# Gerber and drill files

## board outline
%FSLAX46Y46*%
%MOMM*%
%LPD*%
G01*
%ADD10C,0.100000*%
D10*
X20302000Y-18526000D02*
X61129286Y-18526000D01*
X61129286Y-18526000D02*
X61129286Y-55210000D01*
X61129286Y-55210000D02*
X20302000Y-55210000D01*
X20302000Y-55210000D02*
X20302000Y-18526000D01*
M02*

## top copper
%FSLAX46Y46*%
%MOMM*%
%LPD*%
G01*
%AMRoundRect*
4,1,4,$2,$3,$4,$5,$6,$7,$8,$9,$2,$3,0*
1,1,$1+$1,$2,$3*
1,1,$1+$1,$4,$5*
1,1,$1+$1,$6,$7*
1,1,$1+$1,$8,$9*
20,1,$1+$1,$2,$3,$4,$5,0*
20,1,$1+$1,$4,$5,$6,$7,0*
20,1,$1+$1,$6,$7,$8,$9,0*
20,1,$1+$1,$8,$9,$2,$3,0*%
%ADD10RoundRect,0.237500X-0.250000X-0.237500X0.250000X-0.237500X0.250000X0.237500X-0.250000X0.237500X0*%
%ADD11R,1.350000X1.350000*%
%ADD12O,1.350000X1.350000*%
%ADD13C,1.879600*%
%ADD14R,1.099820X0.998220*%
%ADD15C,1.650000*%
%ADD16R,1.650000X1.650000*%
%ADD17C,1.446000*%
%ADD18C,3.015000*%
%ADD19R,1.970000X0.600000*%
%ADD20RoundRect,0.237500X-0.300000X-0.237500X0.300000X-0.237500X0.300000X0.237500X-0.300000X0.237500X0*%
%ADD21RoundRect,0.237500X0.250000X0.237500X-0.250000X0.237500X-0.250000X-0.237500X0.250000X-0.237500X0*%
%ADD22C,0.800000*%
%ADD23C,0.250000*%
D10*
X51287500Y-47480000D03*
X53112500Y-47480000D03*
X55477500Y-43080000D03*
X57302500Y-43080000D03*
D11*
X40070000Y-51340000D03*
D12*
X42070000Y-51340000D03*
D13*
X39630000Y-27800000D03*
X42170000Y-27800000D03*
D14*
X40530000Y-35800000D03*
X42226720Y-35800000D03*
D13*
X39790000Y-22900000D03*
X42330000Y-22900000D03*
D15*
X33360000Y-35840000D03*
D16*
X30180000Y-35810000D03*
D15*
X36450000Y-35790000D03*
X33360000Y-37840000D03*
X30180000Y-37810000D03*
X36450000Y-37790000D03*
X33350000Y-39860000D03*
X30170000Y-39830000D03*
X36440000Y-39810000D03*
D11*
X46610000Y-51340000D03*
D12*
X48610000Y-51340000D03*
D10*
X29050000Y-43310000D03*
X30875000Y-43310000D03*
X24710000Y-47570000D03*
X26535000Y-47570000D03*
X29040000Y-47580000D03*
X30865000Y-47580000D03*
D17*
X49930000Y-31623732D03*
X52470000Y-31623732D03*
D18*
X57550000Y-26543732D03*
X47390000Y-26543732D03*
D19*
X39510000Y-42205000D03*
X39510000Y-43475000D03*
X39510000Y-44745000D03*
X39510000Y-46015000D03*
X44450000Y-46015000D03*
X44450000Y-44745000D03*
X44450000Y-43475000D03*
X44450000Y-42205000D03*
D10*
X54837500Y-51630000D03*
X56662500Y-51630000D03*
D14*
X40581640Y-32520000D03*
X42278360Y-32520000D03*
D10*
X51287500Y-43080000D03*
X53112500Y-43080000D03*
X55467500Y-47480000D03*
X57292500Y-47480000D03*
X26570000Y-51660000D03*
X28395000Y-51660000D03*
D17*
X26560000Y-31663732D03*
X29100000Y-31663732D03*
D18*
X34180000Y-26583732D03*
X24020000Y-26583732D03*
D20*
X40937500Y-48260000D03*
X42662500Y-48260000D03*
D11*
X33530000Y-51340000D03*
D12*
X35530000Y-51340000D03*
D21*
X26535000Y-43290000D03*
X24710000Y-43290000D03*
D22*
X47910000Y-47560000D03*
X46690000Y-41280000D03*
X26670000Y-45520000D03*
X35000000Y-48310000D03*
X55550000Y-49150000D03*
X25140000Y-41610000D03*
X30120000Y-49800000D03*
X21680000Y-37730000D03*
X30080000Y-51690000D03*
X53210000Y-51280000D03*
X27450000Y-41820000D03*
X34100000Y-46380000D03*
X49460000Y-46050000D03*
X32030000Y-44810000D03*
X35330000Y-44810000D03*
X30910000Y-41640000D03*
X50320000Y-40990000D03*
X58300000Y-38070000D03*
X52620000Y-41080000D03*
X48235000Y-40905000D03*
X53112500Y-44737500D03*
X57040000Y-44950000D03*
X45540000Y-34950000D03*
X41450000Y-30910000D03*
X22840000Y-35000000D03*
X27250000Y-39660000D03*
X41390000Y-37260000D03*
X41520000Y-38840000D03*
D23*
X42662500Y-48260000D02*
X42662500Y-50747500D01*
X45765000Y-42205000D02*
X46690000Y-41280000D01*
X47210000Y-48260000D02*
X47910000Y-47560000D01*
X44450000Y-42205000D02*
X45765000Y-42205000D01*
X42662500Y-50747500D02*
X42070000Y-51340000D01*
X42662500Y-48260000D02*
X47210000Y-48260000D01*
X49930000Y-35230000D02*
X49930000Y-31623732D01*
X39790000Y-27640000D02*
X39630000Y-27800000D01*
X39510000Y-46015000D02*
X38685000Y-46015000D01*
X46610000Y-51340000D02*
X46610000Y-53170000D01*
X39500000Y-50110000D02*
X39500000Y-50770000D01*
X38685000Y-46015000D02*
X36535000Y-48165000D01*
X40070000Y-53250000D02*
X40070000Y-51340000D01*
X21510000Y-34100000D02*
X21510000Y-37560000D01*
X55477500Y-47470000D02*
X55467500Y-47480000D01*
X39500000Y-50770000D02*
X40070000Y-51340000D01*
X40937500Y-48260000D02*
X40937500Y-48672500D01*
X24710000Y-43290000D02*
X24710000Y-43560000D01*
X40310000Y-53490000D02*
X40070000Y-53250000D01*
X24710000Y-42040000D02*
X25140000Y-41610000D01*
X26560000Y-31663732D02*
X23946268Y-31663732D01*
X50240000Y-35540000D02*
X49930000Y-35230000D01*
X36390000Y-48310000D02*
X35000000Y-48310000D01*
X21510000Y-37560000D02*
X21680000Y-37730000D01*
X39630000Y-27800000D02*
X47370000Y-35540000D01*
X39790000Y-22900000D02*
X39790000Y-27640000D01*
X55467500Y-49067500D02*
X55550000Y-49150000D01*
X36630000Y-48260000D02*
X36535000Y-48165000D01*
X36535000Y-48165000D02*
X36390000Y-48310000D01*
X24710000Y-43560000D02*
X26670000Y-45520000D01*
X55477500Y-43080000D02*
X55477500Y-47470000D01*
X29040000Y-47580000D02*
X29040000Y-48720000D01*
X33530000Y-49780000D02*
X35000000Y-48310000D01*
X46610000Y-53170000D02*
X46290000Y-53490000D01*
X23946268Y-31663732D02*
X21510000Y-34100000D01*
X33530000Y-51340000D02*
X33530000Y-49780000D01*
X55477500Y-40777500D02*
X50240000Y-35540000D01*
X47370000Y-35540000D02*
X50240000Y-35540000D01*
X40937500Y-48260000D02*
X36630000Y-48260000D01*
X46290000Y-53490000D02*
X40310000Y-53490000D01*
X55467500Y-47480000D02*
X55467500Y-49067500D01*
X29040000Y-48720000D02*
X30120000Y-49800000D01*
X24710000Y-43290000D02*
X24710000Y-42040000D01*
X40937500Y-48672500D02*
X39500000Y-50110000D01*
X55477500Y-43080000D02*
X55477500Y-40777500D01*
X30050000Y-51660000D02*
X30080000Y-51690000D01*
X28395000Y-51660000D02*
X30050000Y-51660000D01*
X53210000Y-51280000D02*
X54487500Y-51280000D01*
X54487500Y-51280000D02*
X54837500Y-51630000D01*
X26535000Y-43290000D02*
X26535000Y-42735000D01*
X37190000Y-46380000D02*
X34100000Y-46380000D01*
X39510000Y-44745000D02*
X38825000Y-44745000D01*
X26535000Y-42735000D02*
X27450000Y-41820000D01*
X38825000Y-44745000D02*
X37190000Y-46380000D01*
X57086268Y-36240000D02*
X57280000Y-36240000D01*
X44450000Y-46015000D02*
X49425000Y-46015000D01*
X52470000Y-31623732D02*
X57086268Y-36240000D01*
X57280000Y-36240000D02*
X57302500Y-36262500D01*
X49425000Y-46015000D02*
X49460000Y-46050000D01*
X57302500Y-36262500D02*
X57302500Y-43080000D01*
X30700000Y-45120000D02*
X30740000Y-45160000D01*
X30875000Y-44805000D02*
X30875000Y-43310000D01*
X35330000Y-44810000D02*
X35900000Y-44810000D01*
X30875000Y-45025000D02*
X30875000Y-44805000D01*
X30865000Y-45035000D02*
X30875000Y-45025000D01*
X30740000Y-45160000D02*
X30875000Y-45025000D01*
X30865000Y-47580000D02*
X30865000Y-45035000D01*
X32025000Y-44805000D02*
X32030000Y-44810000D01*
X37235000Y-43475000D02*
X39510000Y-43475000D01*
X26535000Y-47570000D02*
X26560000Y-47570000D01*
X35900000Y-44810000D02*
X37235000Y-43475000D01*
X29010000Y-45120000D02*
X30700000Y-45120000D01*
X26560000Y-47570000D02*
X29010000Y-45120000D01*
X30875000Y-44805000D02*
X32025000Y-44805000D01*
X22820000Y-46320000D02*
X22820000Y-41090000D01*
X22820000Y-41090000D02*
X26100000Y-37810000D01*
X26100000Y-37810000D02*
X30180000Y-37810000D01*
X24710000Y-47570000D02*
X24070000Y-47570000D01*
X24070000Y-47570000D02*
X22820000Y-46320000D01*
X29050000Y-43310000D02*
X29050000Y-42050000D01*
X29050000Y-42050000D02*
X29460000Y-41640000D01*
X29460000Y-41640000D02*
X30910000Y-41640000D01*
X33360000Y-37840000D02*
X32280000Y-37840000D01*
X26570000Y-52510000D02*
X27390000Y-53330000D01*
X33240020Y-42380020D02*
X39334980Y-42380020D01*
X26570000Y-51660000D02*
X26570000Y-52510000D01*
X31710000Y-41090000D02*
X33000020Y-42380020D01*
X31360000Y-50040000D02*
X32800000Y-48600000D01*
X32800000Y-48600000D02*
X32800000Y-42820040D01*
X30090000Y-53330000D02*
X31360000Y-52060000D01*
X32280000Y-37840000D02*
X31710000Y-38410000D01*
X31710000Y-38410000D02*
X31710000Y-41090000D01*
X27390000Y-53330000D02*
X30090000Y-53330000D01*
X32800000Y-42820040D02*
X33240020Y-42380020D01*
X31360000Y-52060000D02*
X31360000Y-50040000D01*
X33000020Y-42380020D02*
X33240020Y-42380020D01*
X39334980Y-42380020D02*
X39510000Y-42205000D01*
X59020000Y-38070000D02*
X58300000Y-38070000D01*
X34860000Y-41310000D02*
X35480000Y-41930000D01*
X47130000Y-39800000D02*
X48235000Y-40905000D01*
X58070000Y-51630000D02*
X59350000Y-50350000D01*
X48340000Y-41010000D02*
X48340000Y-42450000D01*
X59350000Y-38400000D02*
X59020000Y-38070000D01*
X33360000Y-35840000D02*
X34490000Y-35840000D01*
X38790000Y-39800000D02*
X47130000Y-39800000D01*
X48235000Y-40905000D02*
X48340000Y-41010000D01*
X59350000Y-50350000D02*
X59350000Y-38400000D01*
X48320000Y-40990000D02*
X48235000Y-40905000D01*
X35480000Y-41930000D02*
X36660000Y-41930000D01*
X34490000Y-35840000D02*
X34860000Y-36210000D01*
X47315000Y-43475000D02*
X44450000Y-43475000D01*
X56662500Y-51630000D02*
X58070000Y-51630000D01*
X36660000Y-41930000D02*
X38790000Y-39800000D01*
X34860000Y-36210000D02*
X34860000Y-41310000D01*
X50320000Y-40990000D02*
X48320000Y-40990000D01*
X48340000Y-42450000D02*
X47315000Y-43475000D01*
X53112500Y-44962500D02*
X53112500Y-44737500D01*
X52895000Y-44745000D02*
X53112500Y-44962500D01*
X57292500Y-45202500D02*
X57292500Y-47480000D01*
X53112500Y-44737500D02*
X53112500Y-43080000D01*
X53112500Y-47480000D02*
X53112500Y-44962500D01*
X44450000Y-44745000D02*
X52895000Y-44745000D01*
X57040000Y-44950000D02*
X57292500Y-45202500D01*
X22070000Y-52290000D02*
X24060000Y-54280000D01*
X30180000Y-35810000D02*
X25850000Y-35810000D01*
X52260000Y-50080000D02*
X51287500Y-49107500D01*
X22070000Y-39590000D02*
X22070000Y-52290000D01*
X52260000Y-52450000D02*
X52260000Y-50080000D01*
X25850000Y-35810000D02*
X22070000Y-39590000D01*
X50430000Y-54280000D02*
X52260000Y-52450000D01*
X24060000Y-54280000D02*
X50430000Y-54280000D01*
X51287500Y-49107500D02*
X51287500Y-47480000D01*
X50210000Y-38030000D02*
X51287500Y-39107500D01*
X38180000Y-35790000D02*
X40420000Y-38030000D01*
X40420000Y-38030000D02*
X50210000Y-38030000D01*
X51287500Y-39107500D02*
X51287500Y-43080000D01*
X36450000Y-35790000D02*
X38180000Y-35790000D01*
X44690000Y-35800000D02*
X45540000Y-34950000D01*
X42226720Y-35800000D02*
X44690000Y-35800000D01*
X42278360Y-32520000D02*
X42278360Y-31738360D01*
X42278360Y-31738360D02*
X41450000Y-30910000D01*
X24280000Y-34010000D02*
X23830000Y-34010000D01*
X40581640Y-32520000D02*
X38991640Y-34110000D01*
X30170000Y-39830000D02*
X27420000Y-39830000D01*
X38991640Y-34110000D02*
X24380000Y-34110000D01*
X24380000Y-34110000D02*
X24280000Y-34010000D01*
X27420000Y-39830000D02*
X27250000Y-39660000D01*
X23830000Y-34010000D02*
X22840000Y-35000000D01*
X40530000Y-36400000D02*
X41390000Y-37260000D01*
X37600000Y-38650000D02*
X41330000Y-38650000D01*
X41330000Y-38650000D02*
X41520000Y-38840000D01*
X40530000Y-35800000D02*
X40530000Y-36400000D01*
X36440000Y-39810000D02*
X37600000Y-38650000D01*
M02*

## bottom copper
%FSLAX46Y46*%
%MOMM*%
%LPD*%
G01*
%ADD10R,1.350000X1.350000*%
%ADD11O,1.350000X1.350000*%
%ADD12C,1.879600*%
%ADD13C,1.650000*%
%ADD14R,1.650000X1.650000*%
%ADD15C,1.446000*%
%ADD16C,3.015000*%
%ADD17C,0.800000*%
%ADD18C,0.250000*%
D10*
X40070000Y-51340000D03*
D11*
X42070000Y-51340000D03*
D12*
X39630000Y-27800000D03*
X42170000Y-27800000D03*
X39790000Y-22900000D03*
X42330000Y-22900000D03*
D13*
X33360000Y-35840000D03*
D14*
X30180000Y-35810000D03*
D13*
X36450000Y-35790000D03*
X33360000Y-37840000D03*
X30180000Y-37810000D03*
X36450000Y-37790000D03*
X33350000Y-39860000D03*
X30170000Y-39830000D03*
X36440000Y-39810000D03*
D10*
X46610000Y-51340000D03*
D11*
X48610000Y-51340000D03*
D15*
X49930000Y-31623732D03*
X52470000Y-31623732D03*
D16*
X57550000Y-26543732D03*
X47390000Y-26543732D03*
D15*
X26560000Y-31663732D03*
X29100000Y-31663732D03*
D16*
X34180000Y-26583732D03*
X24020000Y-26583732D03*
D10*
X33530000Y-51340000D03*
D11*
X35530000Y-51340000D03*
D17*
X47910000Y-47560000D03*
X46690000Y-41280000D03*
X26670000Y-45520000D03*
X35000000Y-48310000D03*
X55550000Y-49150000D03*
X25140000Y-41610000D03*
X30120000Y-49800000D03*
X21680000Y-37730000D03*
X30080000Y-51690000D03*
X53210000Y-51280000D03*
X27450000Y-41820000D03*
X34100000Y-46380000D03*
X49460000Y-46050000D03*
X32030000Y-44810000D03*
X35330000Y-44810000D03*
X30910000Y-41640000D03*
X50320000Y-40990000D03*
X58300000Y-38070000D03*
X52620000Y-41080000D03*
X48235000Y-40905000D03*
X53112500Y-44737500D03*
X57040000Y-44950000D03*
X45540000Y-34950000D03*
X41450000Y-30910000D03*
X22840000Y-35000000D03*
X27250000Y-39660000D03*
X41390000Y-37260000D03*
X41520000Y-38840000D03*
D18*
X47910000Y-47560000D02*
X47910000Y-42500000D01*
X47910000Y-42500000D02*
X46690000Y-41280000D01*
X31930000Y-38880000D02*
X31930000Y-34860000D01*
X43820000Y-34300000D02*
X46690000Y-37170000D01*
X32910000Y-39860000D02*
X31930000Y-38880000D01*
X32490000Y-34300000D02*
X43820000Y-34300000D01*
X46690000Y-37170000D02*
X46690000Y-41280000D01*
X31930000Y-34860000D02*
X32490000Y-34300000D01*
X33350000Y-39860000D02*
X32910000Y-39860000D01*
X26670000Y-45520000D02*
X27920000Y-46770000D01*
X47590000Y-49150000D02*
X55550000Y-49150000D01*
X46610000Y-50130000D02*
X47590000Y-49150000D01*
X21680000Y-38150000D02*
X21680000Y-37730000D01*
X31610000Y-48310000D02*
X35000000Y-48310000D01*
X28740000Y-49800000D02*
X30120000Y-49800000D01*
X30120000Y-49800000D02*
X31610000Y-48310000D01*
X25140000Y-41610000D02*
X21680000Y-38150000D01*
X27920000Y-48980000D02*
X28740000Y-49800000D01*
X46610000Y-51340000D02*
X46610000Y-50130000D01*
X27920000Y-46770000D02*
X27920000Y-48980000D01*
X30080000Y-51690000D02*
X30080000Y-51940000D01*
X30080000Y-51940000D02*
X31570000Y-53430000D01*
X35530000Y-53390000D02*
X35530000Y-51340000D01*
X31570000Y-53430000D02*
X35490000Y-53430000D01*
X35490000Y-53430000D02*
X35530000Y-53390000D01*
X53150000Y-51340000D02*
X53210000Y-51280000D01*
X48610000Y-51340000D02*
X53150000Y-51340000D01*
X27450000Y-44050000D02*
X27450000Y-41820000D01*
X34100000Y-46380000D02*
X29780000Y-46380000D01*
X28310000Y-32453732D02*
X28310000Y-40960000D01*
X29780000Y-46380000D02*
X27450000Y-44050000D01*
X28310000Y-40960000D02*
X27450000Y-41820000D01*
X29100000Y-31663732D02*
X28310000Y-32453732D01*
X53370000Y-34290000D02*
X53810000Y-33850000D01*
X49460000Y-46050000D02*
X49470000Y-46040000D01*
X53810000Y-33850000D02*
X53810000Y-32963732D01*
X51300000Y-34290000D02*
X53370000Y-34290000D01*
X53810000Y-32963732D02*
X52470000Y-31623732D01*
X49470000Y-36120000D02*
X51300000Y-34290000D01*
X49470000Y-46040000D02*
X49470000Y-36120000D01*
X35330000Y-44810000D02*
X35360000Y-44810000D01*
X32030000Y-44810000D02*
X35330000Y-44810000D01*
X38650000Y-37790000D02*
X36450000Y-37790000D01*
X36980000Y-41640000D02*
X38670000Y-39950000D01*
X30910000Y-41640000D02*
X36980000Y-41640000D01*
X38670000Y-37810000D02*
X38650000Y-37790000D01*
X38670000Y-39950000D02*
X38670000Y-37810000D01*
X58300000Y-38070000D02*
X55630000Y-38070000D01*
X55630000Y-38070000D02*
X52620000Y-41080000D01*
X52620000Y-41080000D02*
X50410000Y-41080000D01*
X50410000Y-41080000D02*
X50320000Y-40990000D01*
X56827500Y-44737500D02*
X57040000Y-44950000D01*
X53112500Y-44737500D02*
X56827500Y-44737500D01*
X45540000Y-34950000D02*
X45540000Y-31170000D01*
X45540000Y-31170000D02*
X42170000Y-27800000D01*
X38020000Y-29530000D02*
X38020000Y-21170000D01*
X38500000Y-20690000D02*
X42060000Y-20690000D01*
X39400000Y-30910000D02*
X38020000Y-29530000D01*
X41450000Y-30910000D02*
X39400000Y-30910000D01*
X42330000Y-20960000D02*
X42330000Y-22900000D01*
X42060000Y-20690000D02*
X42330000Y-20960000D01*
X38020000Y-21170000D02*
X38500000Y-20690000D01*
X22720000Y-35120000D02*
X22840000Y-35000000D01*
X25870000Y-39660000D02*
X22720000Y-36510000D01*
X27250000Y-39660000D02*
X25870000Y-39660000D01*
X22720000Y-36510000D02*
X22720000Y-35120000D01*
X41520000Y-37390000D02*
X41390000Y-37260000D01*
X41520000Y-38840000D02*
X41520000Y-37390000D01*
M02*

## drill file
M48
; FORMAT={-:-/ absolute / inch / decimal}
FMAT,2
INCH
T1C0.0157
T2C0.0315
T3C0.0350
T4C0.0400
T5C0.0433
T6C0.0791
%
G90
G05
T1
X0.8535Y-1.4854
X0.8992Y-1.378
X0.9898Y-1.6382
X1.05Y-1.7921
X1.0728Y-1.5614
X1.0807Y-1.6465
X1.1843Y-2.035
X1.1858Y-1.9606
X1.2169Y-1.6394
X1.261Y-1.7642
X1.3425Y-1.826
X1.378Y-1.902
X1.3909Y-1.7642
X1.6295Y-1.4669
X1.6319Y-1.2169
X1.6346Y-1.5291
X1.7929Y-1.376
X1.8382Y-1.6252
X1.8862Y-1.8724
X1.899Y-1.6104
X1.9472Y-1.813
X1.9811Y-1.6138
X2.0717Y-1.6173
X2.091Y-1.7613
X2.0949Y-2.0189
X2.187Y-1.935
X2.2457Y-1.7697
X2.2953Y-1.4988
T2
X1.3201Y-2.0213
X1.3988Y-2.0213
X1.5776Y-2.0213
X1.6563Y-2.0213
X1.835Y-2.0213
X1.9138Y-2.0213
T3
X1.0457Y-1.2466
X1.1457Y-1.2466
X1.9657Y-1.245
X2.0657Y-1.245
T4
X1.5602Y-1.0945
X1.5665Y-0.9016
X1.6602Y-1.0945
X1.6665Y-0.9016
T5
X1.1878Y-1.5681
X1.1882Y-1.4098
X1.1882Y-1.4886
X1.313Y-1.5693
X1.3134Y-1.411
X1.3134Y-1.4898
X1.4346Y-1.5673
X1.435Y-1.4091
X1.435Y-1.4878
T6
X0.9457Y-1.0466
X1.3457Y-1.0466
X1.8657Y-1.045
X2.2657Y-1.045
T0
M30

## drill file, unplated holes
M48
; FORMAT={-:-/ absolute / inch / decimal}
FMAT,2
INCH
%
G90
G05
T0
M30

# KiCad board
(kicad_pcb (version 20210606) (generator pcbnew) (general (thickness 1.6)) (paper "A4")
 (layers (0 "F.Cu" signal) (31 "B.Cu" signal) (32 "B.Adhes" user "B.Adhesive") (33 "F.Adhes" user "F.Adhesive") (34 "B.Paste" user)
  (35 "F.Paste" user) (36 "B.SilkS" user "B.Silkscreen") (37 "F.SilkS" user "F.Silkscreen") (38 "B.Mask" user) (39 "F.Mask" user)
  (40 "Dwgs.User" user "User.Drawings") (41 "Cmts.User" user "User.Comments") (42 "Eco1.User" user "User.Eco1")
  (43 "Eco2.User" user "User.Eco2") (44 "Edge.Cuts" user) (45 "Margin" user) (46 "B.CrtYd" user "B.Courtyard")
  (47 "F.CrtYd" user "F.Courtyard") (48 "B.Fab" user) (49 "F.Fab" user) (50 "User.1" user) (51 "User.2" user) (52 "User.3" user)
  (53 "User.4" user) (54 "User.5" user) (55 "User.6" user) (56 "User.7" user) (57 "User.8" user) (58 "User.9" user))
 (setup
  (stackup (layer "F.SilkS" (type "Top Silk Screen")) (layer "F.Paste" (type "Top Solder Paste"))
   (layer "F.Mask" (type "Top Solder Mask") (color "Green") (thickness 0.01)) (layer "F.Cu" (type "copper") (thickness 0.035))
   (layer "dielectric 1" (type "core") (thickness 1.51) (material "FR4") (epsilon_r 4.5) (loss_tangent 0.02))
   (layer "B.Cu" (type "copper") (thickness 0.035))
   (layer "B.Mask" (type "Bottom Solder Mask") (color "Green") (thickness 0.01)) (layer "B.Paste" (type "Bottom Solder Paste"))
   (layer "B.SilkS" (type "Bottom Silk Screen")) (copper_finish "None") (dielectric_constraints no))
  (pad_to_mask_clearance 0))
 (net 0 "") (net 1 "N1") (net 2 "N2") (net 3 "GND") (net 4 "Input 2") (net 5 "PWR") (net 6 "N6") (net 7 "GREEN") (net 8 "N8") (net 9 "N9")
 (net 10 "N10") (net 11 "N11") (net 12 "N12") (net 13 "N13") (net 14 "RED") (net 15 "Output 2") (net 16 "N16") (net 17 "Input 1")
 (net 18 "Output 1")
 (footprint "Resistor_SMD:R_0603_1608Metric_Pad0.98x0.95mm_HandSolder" (layer "F.Cu") (at 52.2 47.48)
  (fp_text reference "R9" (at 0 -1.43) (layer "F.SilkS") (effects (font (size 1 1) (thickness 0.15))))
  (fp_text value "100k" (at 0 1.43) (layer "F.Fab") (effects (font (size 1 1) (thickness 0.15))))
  (pad "1" smd roundrect locked (at -0.9125 0) (size 0.975 0.95) (layers "F.Cu" "F.Paste" "F.Mask") (roundrect_rratio 0.25) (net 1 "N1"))
  (pad "2" smd roundrect locked (at 0.9125 0) (size 0.975 0.95) (layers "F.Cu" "F.Paste" "F.Mask") (roundrect_rratio 0.25) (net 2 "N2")))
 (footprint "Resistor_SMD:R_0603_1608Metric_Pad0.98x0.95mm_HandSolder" (layer "F.Cu") (at 56.39 43.08)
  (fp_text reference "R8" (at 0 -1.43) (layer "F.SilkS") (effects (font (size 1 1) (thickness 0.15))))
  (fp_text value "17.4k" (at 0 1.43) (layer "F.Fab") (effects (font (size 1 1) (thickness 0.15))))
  (pad "1" smd roundrect locked (at -0.9125 0) (size 0.975 0.95) (layers "F.Cu" "F.Paste" "F.Mask") (roundrect_rratio 0.25) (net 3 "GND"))
  (pad "2" smd roundrect locked (at 0.9125 0) (size 0.975 0.95) (layers "F.Cu" "F.Paste" "F.Mask") (roundrect_rratio 0.25) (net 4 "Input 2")))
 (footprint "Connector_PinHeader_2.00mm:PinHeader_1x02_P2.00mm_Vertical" (layer "F.Cu") (at 40.07 51.34 90)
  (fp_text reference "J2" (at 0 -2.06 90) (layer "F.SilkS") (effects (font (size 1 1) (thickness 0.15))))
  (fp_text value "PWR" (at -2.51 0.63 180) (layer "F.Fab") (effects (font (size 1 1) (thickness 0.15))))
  (pad "1" thru_hole rect locked (at 0 0 90) (size 1.35 1.35) (drill 0.8) (layers *.Cu *.Mask) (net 3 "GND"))
  (pad "2" thru_hole oval locked (at 0 2 90) (size 1.35 1.35) (drill 0.8) (layers *.Cu *.Mask) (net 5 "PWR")))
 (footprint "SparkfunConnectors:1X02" (layer "F.Cu") (at 39.63 27.8)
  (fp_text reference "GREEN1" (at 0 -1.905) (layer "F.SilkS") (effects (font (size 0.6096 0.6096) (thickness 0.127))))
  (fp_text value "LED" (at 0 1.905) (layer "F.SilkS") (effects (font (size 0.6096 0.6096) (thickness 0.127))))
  (pad "1" thru_hole circle locked (at 0 0) (size 1.8796 1.8796) (drill 1.016) (layers *.Cu *.Mask) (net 3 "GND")
   (solder_mask_margin 0.1016))
  (pad "2" thru_hole circle locked (at 2.54 0) (size 1.8796 1.8796) (drill 1.016) (layers *.Cu *.Mask) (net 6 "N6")
   (solder_mask_margin 0.1016)))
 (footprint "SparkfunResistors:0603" (layer "F.Cu") (at 41.37836 35.8)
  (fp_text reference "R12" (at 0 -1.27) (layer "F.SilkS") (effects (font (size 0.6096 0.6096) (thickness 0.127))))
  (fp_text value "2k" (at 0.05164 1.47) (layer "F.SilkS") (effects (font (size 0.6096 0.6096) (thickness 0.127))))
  (pad "1" smd rect locked (at -0.84836 0) (size 1.09982 0.99822) (layers "F.Cu" "F.Paste" "F.Mask") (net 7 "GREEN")
   (solder_mask_margin 0.1016))
  (pad "2" smd rect locked (at 0.84836 0) (size 1.09982 0.99822) (layers "F.Cu" "F.Paste" "F.Mask") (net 6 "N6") (solder_mask_margin 0.1016)))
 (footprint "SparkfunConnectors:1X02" (layer "F.Cu") (at 39.79 22.9)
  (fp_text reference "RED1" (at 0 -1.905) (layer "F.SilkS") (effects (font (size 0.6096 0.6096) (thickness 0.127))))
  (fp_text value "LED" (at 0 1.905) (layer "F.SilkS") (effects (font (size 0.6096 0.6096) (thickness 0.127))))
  (pad "1" thru_hole circle locked (at 0 0) (size 1.8796 1.8796) (drill 1.016) (layers *.Cu *.Mask) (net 3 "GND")
   (solder_mask_margin 0.1016))
  (pad "2" thru_hole circle locked (at 2.54 0) (size 1.8796 1.8796) (drill 1.016) (layers *.Cu *.Mask) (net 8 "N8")
   (solder_mask_margin 0.1016)))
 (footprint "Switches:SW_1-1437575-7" (layer "F.Cu") (at 32.68 36.81)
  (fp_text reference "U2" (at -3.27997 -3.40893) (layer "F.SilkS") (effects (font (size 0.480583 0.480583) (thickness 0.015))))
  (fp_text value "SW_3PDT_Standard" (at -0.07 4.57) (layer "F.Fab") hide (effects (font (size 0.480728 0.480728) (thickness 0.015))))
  (pad "1" thru_hole circle locked (at 0.68 -0.97) (size 1.65 1.65) (drill 1.1) (layers *.Cu *.Mask) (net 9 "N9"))
  (pad "2" thru_hole rect locked (at -2.5 -1) (size 1.65 1.65) (drill 1.1) (layers *.Cu *.Mask) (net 1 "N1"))
  (pad "3" thru_hole circle locked (at 3.77 -1.02) (size 1.65 1.65) (drill 1.1) (layers *.Cu *.Mask) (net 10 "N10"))
  (pad "4" thru_hole circle locked (at 0.68 1.03) (size 1.65 1.65) (drill 1.1) (layers *.Cu *.Mask) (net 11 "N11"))
  (pad "5" thru_hole circle locked (at -2.5 1) (size 1.65 1.65) (drill 1.1) (layers *.Cu *.Mask) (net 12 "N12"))
  (pad "6" thru_hole circle locked (at 3.77 0.98) (size 1.65 1.65) (drill 1.1) (layers *.Cu *.Mask) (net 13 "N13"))
  (pad "7" thru_hole circle (at 0.67 3.05) (size 1.65 1.65) (drill 1.1) (layers *.Cu *.Mask) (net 5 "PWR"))
  (pad "8" thru_hole circle (at -2.51 3.02) (size 1.65 1.65) (drill 1.1) (layers *.Cu *.Mask) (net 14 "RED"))
  (pad "9" thru_hole circle (at 3.76 3) (size 1.65 1.65) (drill 1.1) (layers *.Cu *.Mask) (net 7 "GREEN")))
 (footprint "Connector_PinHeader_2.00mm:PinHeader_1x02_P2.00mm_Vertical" (layer "F.Cu") (at 46.61 51.34 90)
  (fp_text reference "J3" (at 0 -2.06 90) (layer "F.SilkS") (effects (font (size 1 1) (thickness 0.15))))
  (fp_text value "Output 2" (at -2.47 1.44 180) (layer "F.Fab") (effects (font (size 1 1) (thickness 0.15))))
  (pad "1" thru_hole rect locked (at 0 0 90) (size 1.35 1.35) (drill 0.8) (layers *.Cu *.Mask) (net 3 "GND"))
  (pad "2" thru_hole oval locked (at 0 2 90) (size 1.35 1.35) (drill 0.8) (layers *.Cu *.Mask) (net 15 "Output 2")))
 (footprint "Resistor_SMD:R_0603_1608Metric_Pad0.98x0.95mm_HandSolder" (layer "F.Cu") (at 29.9625 43.31)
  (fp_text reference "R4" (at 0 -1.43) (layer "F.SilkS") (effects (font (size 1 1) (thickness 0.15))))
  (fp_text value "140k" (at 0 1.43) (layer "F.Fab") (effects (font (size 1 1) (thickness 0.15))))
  (pad "1" smd roundrect locked (at -0.9125 0) (size 0.975 0.95) (layers "F.Cu" "F.Paste" "F.Mask") (roundrect_rratio 0.25) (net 13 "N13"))
  (pad "2" smd roundrect locked (at 0.9125 0) (size 0.975 0.95) (layers "F.Cu" "F.Paste" "F.Mask") (roundrect_rratio 0.25) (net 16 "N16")))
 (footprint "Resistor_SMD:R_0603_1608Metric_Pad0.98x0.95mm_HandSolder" (layer "F.Cu") (at 25.6225 47.57)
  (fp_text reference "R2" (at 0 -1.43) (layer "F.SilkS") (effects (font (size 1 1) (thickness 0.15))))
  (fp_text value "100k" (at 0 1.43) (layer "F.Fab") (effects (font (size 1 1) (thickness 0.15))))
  (pad "1" smd roundrect locked (at -0.9125 0) (size 0.975 0.95) (layers "F.Cu" "F.Paste" "F.Mask") (roundrect_rratio 0.25) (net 12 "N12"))
  (pad "2" smd roundrect locked (at 0.9125 0) (size 0.975 0.95) (layers "F.Cu" "F.Paste" "F.Mask") (roundrect_rratio 0.25) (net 16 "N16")))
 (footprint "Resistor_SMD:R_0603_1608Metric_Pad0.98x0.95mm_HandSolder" (layer "F.Cu") (at 29.9525 47.58)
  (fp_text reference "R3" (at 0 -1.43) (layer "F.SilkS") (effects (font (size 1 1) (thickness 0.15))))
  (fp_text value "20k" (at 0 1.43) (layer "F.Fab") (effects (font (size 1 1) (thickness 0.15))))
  (pad "1" smd roundrect locked (at -0.9125 0) (size 0.975 0.95) (layers "F.Cu" "F.Paste" "F.Mask") (roundrect_rratio 0.25) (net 3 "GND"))
  (pad "2" smd roundrect locked (at 0.9125 0) (size 0.975 0.95) (layers "F.Cu" "F.Paste" "F.Mask") (roundrect_rratio 0.25) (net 16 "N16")))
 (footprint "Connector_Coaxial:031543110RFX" (layer "F.Cu") (at 49.93 31.623732)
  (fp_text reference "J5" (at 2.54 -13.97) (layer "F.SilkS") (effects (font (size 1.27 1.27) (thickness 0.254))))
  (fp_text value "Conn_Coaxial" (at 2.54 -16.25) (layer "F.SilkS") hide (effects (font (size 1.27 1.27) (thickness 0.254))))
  (pad "1" thru_hole circle locked (at 0 0) (size 1.446 1.446) (drill 0.89) (layers *.Cu *.Mask) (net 3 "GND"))
  (pad "2" thru_hole circle locked (at 2.54 0) (size 1.446 1.446) (drill 0.89) (layers *.Cu *.Mask) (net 4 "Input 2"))
  (pad "3" thru_hole circle locked (at 7.62 -5.08) (size 3.015 3.015) (drill 2.01) (layers *.Cu *.Mask))
  (pad "4" thru_hole circle locked (at -2.54 -5.08) (size 3.015 3.015) (drill 2.01) (layers *.Cu *.Mask)))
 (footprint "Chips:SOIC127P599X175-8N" (layer "F.Cu") (at 41.98 44.11)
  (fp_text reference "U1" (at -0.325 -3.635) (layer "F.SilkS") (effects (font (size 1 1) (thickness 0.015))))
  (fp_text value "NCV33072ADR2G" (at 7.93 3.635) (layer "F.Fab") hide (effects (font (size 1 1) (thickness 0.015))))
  (pad "1" smd rect locked (at -2.47 -1.905) (size 1.97 0.6) (layers "F.Cu" "F.Paste" "F.Mask") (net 11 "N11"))
  (pad "2" smd rect locked (at -2.47 -0.635) (size 1.97 0.6) (layers "F.Cu" "F.Paste" "F.Mask") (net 16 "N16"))
  (pad "3" smd rect locked (at -2.47 0.635) (size 1.97 0.6) (layers "F.Cu" "F.Paste" "F.Mask") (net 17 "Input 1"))
  (pad "4" smd rect locked (at -2.47 1.905) (size 1.97 0.6) (layers "F.Cu" "F.Paste" "F.Mask") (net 3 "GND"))
  (pad "5" smd rect locked (at 2.47 1.905) (size 1.97 0.6) (layers "F.Cu" "F.Paste" "F.Mask") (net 4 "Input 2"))
  (pad "6" smd rect locked (at 2.47 0.635) (size 1.97 0.6) (layers "F.Cu" "F.Paste" "F.Mask") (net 2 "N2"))
  (pad "7" smd rect locked (at 2.47 -0.635) (size 1.97 0.6) (layers "F.Cu" "F.Paste" "F.Mask") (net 9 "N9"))
  (pad "8" smd rect locked (at 2.47 -1.905) (size 1.97 0.6) (layers "F.Cu" "F.Paste" "F.Mask") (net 5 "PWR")))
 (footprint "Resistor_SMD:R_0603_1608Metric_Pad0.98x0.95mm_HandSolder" (layer "F.Cu") (at 55.75 51.63)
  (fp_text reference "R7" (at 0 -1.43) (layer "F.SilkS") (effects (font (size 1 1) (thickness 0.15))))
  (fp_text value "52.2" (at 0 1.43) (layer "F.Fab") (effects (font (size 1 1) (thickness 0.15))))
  (pad "1" smd roundrect locked (at -0.9125 0) (size 0.975 0.95) (layers "F.Cu" "F.Paste" "F.Mask") (roundrect_rratio 0.25)
   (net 15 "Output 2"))
  (pad "2" smd roundrect locked (at 0.9125 0) (size 0.975 0.95) (layers "F.Cu" "F.Paste" "F.Mask") (roundrect_rratio 0.25) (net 9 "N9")))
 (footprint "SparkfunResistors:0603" (layer "F.Cu") (at 41.43 32.52)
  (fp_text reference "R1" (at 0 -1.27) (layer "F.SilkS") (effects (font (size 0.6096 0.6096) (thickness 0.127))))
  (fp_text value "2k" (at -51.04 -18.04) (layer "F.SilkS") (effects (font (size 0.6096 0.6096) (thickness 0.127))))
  (pad "1" smd rect locked (at -0.84836 0) (size 1.09982 0.99822) (layers "F.Cu" "F.Paste" "F.Mask") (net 14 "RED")
   (solder_mask_margin 0.1016))
  (pad "2" smd rect locked (at 0.84836 0) (size 1.09982 0.99822) (layers "F.Cu" "F.Paste" "F.Mask") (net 8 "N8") (solder_mask_margin 0.1016)))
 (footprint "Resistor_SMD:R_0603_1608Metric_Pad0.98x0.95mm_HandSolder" (layer "F.Cu") (at 52.2 43.08)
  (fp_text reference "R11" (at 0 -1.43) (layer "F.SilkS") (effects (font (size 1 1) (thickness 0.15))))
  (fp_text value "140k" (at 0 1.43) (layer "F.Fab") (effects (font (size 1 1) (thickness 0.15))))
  (pad "1" smd roundrect locked (at -0.9125 0) (size 0.975 0.95) (layers "F.Cu" "F.Paste" "F.Mask") (roundrect_rratio 0.25) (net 10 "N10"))
  (pad "2" smd roundrect locked (at 0.9125 0) (size 0.975 0.95) (layers "F.Cu" "F.Paste" "F.Mask") (roundrect_rratio 0.25) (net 2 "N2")))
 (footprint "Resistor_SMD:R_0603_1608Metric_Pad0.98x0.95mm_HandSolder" (layer "F.Cu") (at 56.38 47.48)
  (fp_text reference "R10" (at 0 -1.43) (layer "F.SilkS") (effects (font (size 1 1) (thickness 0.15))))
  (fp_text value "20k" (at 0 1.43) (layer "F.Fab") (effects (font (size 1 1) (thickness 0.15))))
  (pad "1" smd roundrect locked (at -0.9125 0) (size 0.975 0.95) (layers "F.Cu" "F.Paste" "F.Mask") (roundrect_rratio 0.25) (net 3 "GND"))
  (pad "2" smd roundrect locked (at 0.9125 0) (size 0.975 0.95) (layers "F.Cu" "F.Paste" "F.Mask") (roundrect_rratio 0.25) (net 2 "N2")))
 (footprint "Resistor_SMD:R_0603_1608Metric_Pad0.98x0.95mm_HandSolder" (layer "F.Cu") (at 27.4825 51.66)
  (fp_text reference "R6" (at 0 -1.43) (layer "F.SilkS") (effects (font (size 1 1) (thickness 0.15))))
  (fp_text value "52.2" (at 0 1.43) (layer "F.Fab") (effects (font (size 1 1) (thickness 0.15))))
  (pad "1" smd roundrect locked (at -0.9125 0) (size 0.975 0.95) (layers "F.Cu" "F.Paste" "F.Mask") (roundrect_rratio 0.25) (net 11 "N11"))
  (pad "2" smd roundrect locked (at 0.9125 0) (size 0.975 0.95) (layers "F.Cu" "F.Paste" "F.Mask") (roundrect_rratio 0.25)
   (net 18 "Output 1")))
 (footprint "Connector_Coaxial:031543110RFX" (layer "F.Cu") (at 26.56 31.663732)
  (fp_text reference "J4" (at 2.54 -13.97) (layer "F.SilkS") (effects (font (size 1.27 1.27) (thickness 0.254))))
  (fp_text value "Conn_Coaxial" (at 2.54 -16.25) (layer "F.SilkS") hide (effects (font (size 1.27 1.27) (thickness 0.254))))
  (pad "1" thru_hole circle locked (at 0 0) (size 1.446 1.446) (drill 0.89) (layers *.Cu *.Mask) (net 3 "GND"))
  (pad "2" thru_hole circle locked (at 2.54 0) (size 1.446 1.446) (drill 0.89) (layers *.Cu *.Mask) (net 17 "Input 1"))
  (pad "3" thru_hole circle locked (at 7.62 -5.08) (size 3.015 3.015) (drill 2.01) (layers *.Cu *.Mask))
  (pad "4" thru_hole circle locked (at -2.54 -5.08) (size 3.015 3.015) (drill 2.01) (layers *.Cu *.Mask)))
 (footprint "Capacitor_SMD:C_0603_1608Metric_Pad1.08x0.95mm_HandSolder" (layer "F.Cu") (at 41.8 48.26)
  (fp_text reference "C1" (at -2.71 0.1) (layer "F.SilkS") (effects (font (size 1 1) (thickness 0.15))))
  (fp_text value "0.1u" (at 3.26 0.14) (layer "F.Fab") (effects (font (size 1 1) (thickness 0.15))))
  (pad "1" smd roundrect locked (at -0.8625 0) (size 1.075 0.95) (layers "F.Cu" "F.Paste" "F.Mask") (roundrect_rratio 0.25) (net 3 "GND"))
  (pad "2" smd roundrect locked (at 0.8625 0) (size 1.075 0.95) (layers "F.Cu" "F.Paste" "F.Mask") (roundrect_rratio 0.25) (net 5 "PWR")))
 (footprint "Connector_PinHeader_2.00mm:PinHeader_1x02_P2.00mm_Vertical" (layer "F.Cu") (at 33.53 51.34 90)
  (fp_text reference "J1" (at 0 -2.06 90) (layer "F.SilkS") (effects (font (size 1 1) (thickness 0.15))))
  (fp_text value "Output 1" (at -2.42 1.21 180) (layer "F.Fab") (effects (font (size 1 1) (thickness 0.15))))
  (pad "1" thru_hole rect locked (at 0 0 90) (size 1.35 1.35) (drill 0.8) (layers *.Cu *.Mask) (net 3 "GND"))
  (pad "2" thru_hole oval locked (at 0 2 90) (size 1.35 1.35) (drill 0.8) (layers *.Cu *.Mask) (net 18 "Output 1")))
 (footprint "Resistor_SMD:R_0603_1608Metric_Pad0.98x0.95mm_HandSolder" (layer "F.Cu") (at 25.6225 43.29 180)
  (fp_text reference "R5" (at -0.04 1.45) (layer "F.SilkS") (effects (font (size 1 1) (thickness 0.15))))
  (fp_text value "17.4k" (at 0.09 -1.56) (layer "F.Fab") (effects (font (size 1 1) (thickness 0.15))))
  (pad "1" smd roundrect locked (at -0.9125 0 180) (size 0.975 0.95) (layers "F.Cu" "F.Paste" "F.Mask") (roundrect_rratio 0.25)
   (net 17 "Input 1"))
  (pad "2" smd roundrect locked (at 0.9125 0 180) (size 0.975 0.95) (layers "F.Cu" "F.Paste" "F.Mask") (roundrect_rratio 0.25) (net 3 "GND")))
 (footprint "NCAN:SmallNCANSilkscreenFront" (layer "B.Cu") (at 41.418 41.894 180)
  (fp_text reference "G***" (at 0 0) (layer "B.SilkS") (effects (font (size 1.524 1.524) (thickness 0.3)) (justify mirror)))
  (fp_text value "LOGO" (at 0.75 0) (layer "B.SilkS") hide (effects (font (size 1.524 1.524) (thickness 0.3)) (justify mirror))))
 (gr_rect (start 20.302 18.526) (end 61.129286 55.21) (layer "Edge.Cuts") (width 0.1) (fill none))
 (segment (start 42.6625 48.26) (end 42.6625 50.7475) (width 0.25) (layer "F.Cu") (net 5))
 (segment (start 45.765 42.205) (end 46.69 41.28) (width 0.25) (layer "F.Cu") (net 5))
 (segment (start 47.21 48.26) (end 47.91 47.56) (width 0.25) (layer "F.Cu") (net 5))
 (segment (start 44.45 42.205) (end 45.765 42.205) (width 0.25) (layer "F.Cu") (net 5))
 (segment (start 42.6625 50.7475) (end 42.07 51.34) (width 0.25) (layer "F.Cu") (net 5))
 (segment (start 42.6625 48.26) (end 47.21 48.26) (width 0.25) (layer "F.Cu") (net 5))
 (via (at 47.91 47.56) (size 0.8) (drill 0.4) (layers "F.Cu" "B.Cu") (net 5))
 (via (at 46.69 41.28) (size 0.8) (drill 0.4) (layers "F.Cu" "B.Cu") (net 5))
 (segment (start 47.91 47.56) (end 47.91 42.5) (width 0.25) (layer "B.Cu") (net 5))
 (segment (start 47.91 42.5) (end 46.69 41.28) (width 0.25) (layer "B.Cu") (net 5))
 (segment (start 31.93 38.88) (end 31.93 34.86) (width 0.25) (layer "B.Cu") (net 5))
 (segment (start 43.82 34.3) (end 46.69 37.17) (width 0.25) (layer "B.Cu") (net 5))
 (segment (start 32.91 39.86) (end 31.93 38.88) (width 0.25) (layer "B.Cu") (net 5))
 (segment (start 32.49 34.3) (end 43.82 34.3) (width 0.25) (layer "B.Cu") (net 5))
 (segment (start 46.69 37.17) (end 46.69 41.28) (width 0.25) (layer "B.Cu") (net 5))
 (segment (start 31.93 34.86) (end 32.49 34.3) (width 0.25) (layer "B.Cu") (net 5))
 (segment (start 33.35 39.86) (end 32.91 39.86) (width 0.25) (layer "B.Cu") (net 5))
 (segment (start 49.93 35.23) (end 49.93 31.623732) (width 0.25) (layer "F.Cu") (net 3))
 (segment (start 39.79 27.64) (end 39.63 27.8) (width 0.25) (layer "F.Cu") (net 3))
 (segment (start 39.51 46.015) (end 38.685 46.015) (width 0.25) (layer "F.Cu") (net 3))
 (segment (start 46.61 51.34) (end 46.61 53.17) (width 0.25) (layer "F.Cu") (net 3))
 (segment (start 39.5 50.11) (end 39.5 50.77) (width 0.25) (layer "F.Cu") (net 3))
 (segment (start 38.685 46.015) (end 36.535 48.165) (width 0.25) (layer "F.Cu") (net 3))
 (segment (start 40.07 53.25) (end 40.07 51.34) (width 0.25) (layer "F.Cu") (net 3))
 (segment (start 21.51 34.1) (end 21.51 37.56) (width 0.25) (layer "F.Cu") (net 3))
 (segment (start 55.4775 47.47) (end 55.4675 47.48) (width 0.25) (layer "F.Cu") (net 3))
 (segment (start 39.5 50.77) (end 40.07 51.34) (width 0.25) (layer "F.Cu") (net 3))
 (segment (start 40.9375 48.26) (end 40.9375 48.6725) (width 0.25) (layer "F.Cu") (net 3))
 (segment (start 24.71 43.29) (end 24.71 43.56) (width 0.25) (layer "F.Cu") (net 3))
 (segment (start 40.31 53.49) (end 40.07 53.25) (width 0.25) (layer "F.Cu") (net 3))
 (segment (start 24.71 42.04) (end 25.14 41.61) (width 0.25) (layer "F.Cu") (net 3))
 (segment (start 26.56 31.663732) (end 23.946268 31.663732) (width 0.25) (layer "F.Cu") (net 3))
 (segment (start 50.24 35.54) (end 49.93 35.23) (width 0.25) (layer "F.Cu") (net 3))
 (segment (start 36.39 48.31) (end 35 48.31) (width 0.25) (layer "F.Cu") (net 3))
 (segment (start 21.51 37.56) (end 21.68 37.73) (width 0.25) (layer "F.Cu") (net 3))
 (segment (start 39.63 27.8) (end 47.37 35.54) (width 0.25) (layer "F.Cu") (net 3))
 (segment (start 39.79 22.9) (end 39.79 27.64) (width 0.25) (layer "F.Cu") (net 3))
 (segment (start 55.4675 49.0675) (end 55.55 49.15) (width 0.25) (layer "F.Cu") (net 3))
 (segment (start 36.63 48.26) (end 36.535 48.165) (width 0.25) (layer "F.Cu") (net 3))
 (segment (start 36.535 48.165) (end 36.39 48.31) (width 0.25) (layer "F.Cu") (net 3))
 (segment (start 24.71 43.56) (end 26.67 45.52) (width 0.25) (layer "F.Cu") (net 3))
 (segment (start 55.4775 43.08) (end 55.4775 47.47) (width 0.25) (layer "F.Cu") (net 3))
 (segment (start 29.04 47.58) (end 29.04 48.72) (width 0.25) (layer "F.Cu") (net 3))
 (segment (start 33.53 49.78) (end 35 48.31) (width 0.25) (layer "F.Cu") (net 3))
 (segment (start 46.61 53.17) (end 46.29 53.49) (width 0.25) (layer "F.Cu") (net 3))
 (segment (start 23.946268 31.663732) (end 21.51 34.1) (width 0.25) (layer "F.Cu") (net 3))
 (segment (start 33.53 51.34) (end 33.53 49.78) (width 0.25) (layer "F.Cu") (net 3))
 (segment (start 55.4775 40.7775) (end 50.24 35.54) (width 0.25) (layer "F.Cu") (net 3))
 (segment (start 47.37 35.54) (end 50.24 35.54) (width 0.25) (layer "F.Cu") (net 3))
 (segment (start 40.9375 48.26) (end 36.63 48.26) (width 0.25) (layer "F.Cu") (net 3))
 (segment (start 46.29 53.49) (end 40.31 53.49) (width 0.25) (layer "F.Cu") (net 3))
 (segment (start 55.4675 47.48) (end 55.4675 49.0675) (width 0.25) (layer "F.Cu") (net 3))
 (segment (start 29.04 48.72) (end 30.12 49.8) (width 0.25) (layer "F.Cu") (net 3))
 (segment (start 24.71 43.29) (end 24.71 42.04) (width 0.25) (layer "F.Cu") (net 3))
 (segment (start 40.9375 48.6725) (end 39.5 50.11) (width 0.25) (layer "F.Cu") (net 3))
 (segment (start 55.4775 43.08) (end 55.4775 40.7775) (width 0.25) (layer "F.Cu") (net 3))
 (via (at 26.67 45.52) (size 0.8) (drill 0.4) (layers "F.Cu" "B.Cu") (free) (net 3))
 (via (at 35 48.31) (size 0.8) (drill 0.4) (layers "F.Cu" "B.Cu") (free) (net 3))
 (via (at 55.55 49.15) (size 0.8) (drill 0.4) (layers "F.Cu" "B.Cu") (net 3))
 (via (at 25.14 41.61) (size 0.8) (drill 0.4) (layers "F.Cu" "B.Cu") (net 3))
 (via (at 30.12 49.8) (size 0.8) (drill 0.4) (layers "F.Cu" "B.Cu") (free) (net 3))
 (via (at 21.68 37.73) (size 0.8) (drill 0.4) (layers "F.Cu" "B.Cu") (free) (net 3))
 (segment (start 26.67 45.52) (end 27.92 46.77) (width 0.25) (layer "B.Cu") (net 3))
 (segment (start 47.59 49.15) (end 55.55 49.15) (width 0.25) (layer "B.Cu") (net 3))
 (segment (start 46.61 50.13) (end 47.59 49.15) (width 0.25) (layer "B.Cu") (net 3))
 (segment (start 21.68 38.15) (end 21.68 37.73) (width 0.25) (layer "B.Cu") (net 3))
 (segment (start 31.61 48.31) (end 35 48.31) (width 0.25) (layer "B.Cu") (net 3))
 (segment (start 28.74 49.8) (end 30.12 49.8) (width 0.25) (layer "B.Cu") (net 3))
 (segment (start 30.12 49.8) (end 31.61 48.31) (width 0.25) (layer "B.Cu") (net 3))
 (segment (start 25.14 41.61) (end 21.68 38.15) (width 0.25) (layer "B.Cu") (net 3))
 (segment (start 27.92 48.98) (end 28.74 49.8) (width 0.25) (layer "B.Cu") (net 3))
 (segment (start 46.61 51.34) (end 46.61 50.13) (width 0.25) (layer "B.Cu") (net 3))
 (segment (start 27.92 46.77) (end 27.92 48.98) (width 0.25) (layer "B.Cu") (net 3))
 (segment (start 30.05 51.66) (end 30.08 51.69) (width 0.25) (layer "F.Cu") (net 18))
 (segment (start 28.395 51.66) (end 30.05 51.66) (width 0.25) (layer "F.Cu") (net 18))
 (via (at 30.08 51.69) (size 0.8) (drill 0.4) (layers "F.Cu" "B.Cu") (free) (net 18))
 (segment (start 30.08 51.69) (end 30.08 51.94) (width 0.25) (layer "B.Cu") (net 18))
 (segment (start 30.08 51.94) (end 31.57 53.43) (width 0.25) (layer "B.Cu") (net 18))
 (segment (start 35.53 53.39) (end 35.53 51.34) (width 0.25) (layer "B.Cu") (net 18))
 (segment (start 31.57 53.43) (end 35.49 53.43) (width 0.25) (layer "B.Cu") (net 18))
 (segment (start 35.49 53.43) (end 35.53 53.39) (width 0.25) (layer "B.Cu") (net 18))
 (segment (start 53.21 51.28) (end 54.4875 51.28) (width 0.25) (layer "F.Cu") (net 15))
 (segment (start 54.4875 51.28) (end 54.8375 51.63) (width 0.25) (layer "F.Cu") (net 15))
 (via (at 53.21 51.28) (size 0.8) (drill 0.4) (layers "F.Cu" "B.Cu") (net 15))
 (segment (start 53.15 51.34) (end 53.21 51.28) (width 0.25) (layer "B.Cu") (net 15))
 (segment (start 48.61 51.34) (end 53.15 51.34) (width 0.25) (layer "B.Cu") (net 15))
 (segment (start 26.535 43.29) (end 26.535 42.735) (width 0.25) (layer "F.Cu") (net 17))
 (segment (start 37.19 46.38) (end 34.1 46.38) (width 0.25) (layer "F.Cu") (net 17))
 (segment (start 39.51 44.745) (end 38.825 44.745) (width 0.25) (layer "F.Cu") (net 17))
 (segment (start 26.535 42.735) (end 27.45 41.82) (width 0.25) (layer "F.Cu") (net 17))
 (segment (start 38.825 44.745) (end 37.19 46.38) (width 0.25) (layer "F.Cu") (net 17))
 (via (at 27.45 41.82) (size 0.8) (drill 0.4) (layers "F.Cu" "B.Cu") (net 17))
 (via (at 34.1 46.38) (size 0.8) (drill 0.4) (layers "F.Cu" "B.Cu") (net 17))
 (segment (start 27.45 44.05) (end 27.45 41.82) (width 0.25) (layer "B.Cu") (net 17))
 (segment (start 34.1 46.38) (end 29.78 46.38) (width 0.25) (layer "B.Cu") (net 17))
 (segment (start 28.31 32.453732) (end 28.31 40.96) (width 0.25) (layer "B.Cu") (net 17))
 (segment (start 29.78 46.38) (end 27.45 44.05) (width 0.25) (layer "B.Cu") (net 17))
 (segment (start 28.31 40.96) (end 27.45 41.82) (width 0.25) (layer "B.Cu") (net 17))
 (segment (start 29.1 31.663732) (end 28.31 32.453732) (width 0.25) (layer "B.Cu") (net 17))
 (segment (start 57.086268 36.24) (end 57.28 36.24) (width 0.25) (layer "F.Cu") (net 4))
 (segment (start 44.45 46.015) (end 49.425 46.015) (width 0.25) (layer "F.Cu") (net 4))
 (segment (start 52.47 31.623732) (end 57.086268 36.24) (width 0.25) (layer "F.Cu") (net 4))
 (segment (start 57.28 36.24) (end 57.3025 36.2625) (width 0.25) (layer "F.Cu") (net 4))
 (segment (start 49.425 46.015) (end 49.46 46.05) (width 0.25) (layer "F.Cu") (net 4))
 (segment (start 57.3025 36.2625) (end 57.3025 43.08) (width 0.25) (layer "F.Cu") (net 4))
 (via (at 49.46 46.05) (size 0.8) (drill 0.4) (layers "F.Cu" "B.Cu") (free) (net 4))
 (segment (start 53.37 34.29) (end 53.81 33.85) (width 0.25) (layer "B.Cu") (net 4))
 (segment (start 49.46 46.05) (end 49.47 46.04) (width 0.25) (layer "B.Cu") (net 4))
 (segment (start 53.81 33.85) (end 53.81 32.963732) (width 0.25) (layer "B.Cu") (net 4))
 (segment (start 51.3 34.29) (end 53.37 34.29) (width 0.25) (layer "B.Cu") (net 4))
 (segment (start 53.81 32.963732) (end 52.47 31.623732) (width 0.25) (layer "B.Cu") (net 4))
 (segment (start 49.47 36.12) (end 51.3 34.29) (width 0.25) (layer "B.Cu") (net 4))
 (segment (start 49.47 46.04) (end 49.47 36.12) (width 0.25) (layer "B.Cu") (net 4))
 (segment (start 30.7 45.12) (end 30.74 45.16) (width 0.25) (layer "F.Cu") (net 16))
 (segment (start 30.875 44.805) (end 30.875 43.31) (width 0.25) (layer "F.Cu") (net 16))
 (segment (start 35.33 44.81) (end 35.9 44.81) (width 0.25) (layer "F.Cu") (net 16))
 (segment (start 30.875 45.025) (end 30.875 44.805) (width 0.25) (layer "F.Cu") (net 16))
 (segment (start 30.865 45.035) (end 30.875 45.025) (width 0.25) (layer "F.Cu") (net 16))
 (segment (start 30.74 45.16) (end 30.875 45.025) (width 0.25) (layer "F.Cu") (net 16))
 (segment (start 30.865 47.58) (end 30.865 45.035) (width 0.25) (layer "F.Cu") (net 16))
 (segment (start 32.025 44.805) (end 32.03 44.81) (width 0.25) (layer "F.Cu") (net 16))
 (segment (start 37.235 43.475) (end 39.51 43.475) (width 0.25) (layer "F.Cu") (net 16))
 (segment (start 26.535 47.57) (end 26.56 47.57) (width 0.25) (layer "F.Cu") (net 16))
 (segment (start 35.9 44.81) (end 37.235 43.475) (width 0.25) (layer "F.Cu") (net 16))
 (segment (start 29.01 45.12) (end 30.7 45.12) (width 0.25) (layer "F.Cu") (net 16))
 (segment (start 26.56 47.57) (end 29.01 45.12) (width 0.25) (layer "F.Cu") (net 16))
 (segment (start 30.875 44.805) (end 32.025 44.805) (width 0.25) (layer "F.Cu") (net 16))
 (via (at 32.03 44.81) (size 0.8) (drill 0.4) (layers "F.Cu" "B.Cu") (free) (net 16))
 (via (at 35.33 44.81) (size 0.8) (drill 0.4) (layers "F.Cu" "B.Cu") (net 16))
 (segment (start 35.33 44.81) (end 35.36 44.81) (width 0.25) (layer "B.Cu") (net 16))
 (segment (start 32.03 44.81) (end 35.33 44.81) (width 0.25) (layer "B.Cu") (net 16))
 (segment (start 22.82 46.32) (end 22.82 41.09) (width 0.25) (layer "F.Cu") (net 12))
 (segment (start 22.82 41.09) (end 26.1 37.81) (width 0.25) (layer "F.Cu") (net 12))
 (segment (start 26.1 37.81) (end 30.18 37.81) (width 0.25) (layer "F.Cu") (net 12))
 (segment (start 24.71 47.57) (end 24.07 47.57) (width 0.25) (layer "F.Cu") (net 12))
 (segment (start 24.07 47.57) (end 22.82 46.32) (width 0.25) (layer "F.Cu") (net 12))
 (segment (start 29.05 43.31) (end 29.05 42.05) (width 0.25) (layer "F.Cu") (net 13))
 (segment (start 29.05 42.05) (end 29.46 41.64) (width 0.25) (layer "F.Cu") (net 13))
 (segment (start 29.46 41.64) (end 30.91 41.64) (width 0.25) (layer "F.Cu") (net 13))
 (via (at 30.91 41.64) (size 0.8) (drill 0.4) (layers "F.Cu" "B.Cu") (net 13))
 (segment (start 38.65 37.79) (end 36.45 37.79) (width 0.25) (layer "B.Cu") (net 13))
 (segment (start 36.98 41.64) (end 38.67 39.95) (width 0.25) (layer "B.Cu") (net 13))
 (segment (start 30.91 41.64) (end 36.98 41.64) (width 0.25) (layer "B.Cu") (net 13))
 (segment (start 38.67 37.81) (end 38.65 37.79) (width 0.25) (layer "B.Cu") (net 13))
 (segment (start 38.67 39.95) (end 38.67 37.81) (width 0.25) (layer "B.Cu") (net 13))
 (segment (start 33.36 37.84) (end 32.28 37.84) (width 0.25) (layer "F.Cu") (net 11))
 (segment (start 26.57 52.51) (end 27.39 53.33) (width 0.25) (layer "F.Cu") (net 11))
 (segment (start 33.24002 42.38002) (end 39.33498 42.38002) (width 0.25) (layer "F.Cu") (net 11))
 (segment (start 26.57 51.66) (end 26.57 52.51) (width 0.25) (layer "F.Cu") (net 11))
 (segment (start 31.71 41.09) (end 33.00002 42.38002) (width 0.25) (layer "F.Cu") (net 11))
 (segment (start 31.36 50.04) (end 32.8 48.6) (width 0.25) (layer "F.Cu") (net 11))
 (segment (start 32.8 48.6) (end 32.8 42.82004) (width 0.25) (layer "F.Cu") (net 11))
 (segment (start 30.09 53.33) (end 31.36 52.06) (width 0.25) (layer "F.Cu") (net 11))
 (segment (start 32.28 37.84) (end 31.71 38.41) (width 0.25) (layer "F.Cu") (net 11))
 (segment (start 31.71 38.41) (end 31.71 41.09) (width 0.25) (layer "F.Cu") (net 11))
 (segment (start 27.39 53.33) (end 30.09 53.33) (width 0.25) (layer "F.Cu") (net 11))
 (segment (start 32.8 42.82004) (end 33.24002 42.38002) (width 0.25) (layer "F.Cu") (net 11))
 (segment (start 31.36 52.06) (end 31.36 50.04) (width 0.25) (layer "F.Cu") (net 11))
 (segment (start 33.00002 42.38002) (end 33.24002 42.38002) (width 0.25) (layer "F.Cu") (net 11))
 (segment (start 39.33498 42.38002) (end 39.51 42.205) (width 0.25) (layer "F.Cu") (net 11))
 (segment (start 59.02 38.07) (end 58.3 38.07) (width 0.25) (layer "F.Cu") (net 9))
 (segment (start 34.86 41.31) (end 35.48 41.93) (width 0.25) (layer "F.Cu") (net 9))
 (segment (start 47.13 39.8) (end 48.235 40.905) (width 0.25) (layer "F.Cu") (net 9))
 (segment (start 58.07 51.63) (end 59.35 50.35) (width 0.25) (layer "F.Cu") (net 9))
 (segment (start 48.34 41.01) (end 48.34 42.45) (width 0.25) (layer "F.Cu") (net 9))
 (segment (start 59.35 38.4) (end 59.02 38.07) (width 0.25) (layer "F.Cu") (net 9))
 (segment (start 33.36 35.84) (end 34.49 35.84) (width 0.25) (layer "F.Cu") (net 9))
 (segment (start 38.79 39.8) (end 47.13 39.8) (width 0.25) (layer "F.Cu") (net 9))
 (segment (start 48.235 40.905) (end 48.34 41.01) (width 0.25) (layer "F.Cu") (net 9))
 (segment (start 59.35 50.35) (end 59.35 38.4) (width 0.25) (layer "F.Cu") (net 9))
 (segment (start 48.32 40.99) (end 48.235 40.905) (width 0.25) (layer "F.Cu") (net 9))
 (segment (start 35.48 41.93) (end 36.66 41.93) (width 0.25) (layer "F.Cu") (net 9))
 (segment (start 34.49 35.84) (end 34.86 36.21) (width 0.25) (layer "F.Cu") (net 9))
 (segment (start 47.315 43.475) (end 44.45 43.475) (width 0.25) (layer "F.Cu") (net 9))
 (segment (start 56.6625 51.63) (end 58.07 51.63) (width 0.25) (layer "F.Cu") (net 9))
 (segment (start 36.66 41.93) (end 38.79 39.8) (width 0.25) (layer "F.Cu") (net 9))
 (segment (start 34.86 36.21) (end 34.86 41.31) (width 0.25) (layer "F.Cu") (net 9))
 (segment (start 50.32 40.99) (end 48.32 40.99) (width 0.25) (layer "F.Cu") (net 9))
 (segment (start 48.34 42.45) (end 47.315 43.475) (width 0.25) (layer "F.Cu") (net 9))
 (via (at 50.32 40.99) (size 0.8) (drill 0.4) (layers "F.Cu" "B.Cu") (free) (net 9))
 (via (at 58.3 38.07) (size 0.8) (drill 0.4) (layers "F.Cu" "B.Cu") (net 9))
 (via (at 52.62 41.08) (size 0.8) (drill 0.4) (layers "F.Cu" "B.Cu") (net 9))
 (via (at 48.235 40.905) (size 0.8) (drill 0.4) (layers "F.Cu" "B.Cu") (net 9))
 (segment (start 58.3 38.07) (end 55.63 38.07) (width 0.25) (layer "B.Cu") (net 9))
 (segment (start 55.63 38.07) (end 52.62 41.08) (width 0.25) (layer "B.Cu") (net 9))
 (segment (start 52.62 41.08) (end 50.41 41.08) (width 0.25) (layer "B.Cu") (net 9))
 (segment (start 50.41 41.08) (end 50.32 40.99) (width 0.25) (layer "B.Cu") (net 9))
 (segment (start 53.1125 44.9625) (end 53.1125 44.7375) (width 0.25) (layer "F.Cu") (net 2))
 (segment (start 52.895 44.745) (end 53.1125 44.9625) (width 0.25) (layer "F.Cu") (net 2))
 (segment (start 57.2925 45.2025) (end 57.2925 47.48) (width 0.25) (layer "F.Cu") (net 2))
 (segment (start 53.1125 44.7375) (end 53.1125 43.08) (width 0.25) (layer "F.Cu") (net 2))
 (segment (start 53.1125 47.48) (end 53.1125 44.9625) (width 0.25) (layer "F.Cu") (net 2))
 (segment (start 44.45 44.745) (end 52.895 44.745) (width 0.25) (layer "F.Cu") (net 2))
 (segment (start 57.04 44.95) (end 57.2925 45.2025) (width 0.25) (layer "F.Cu") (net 2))
 (via (at 53.1125 44.7375) (size 0.8) (drill 0.4) (layers "F.Cu" "B.Cu") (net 2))
 (via (at 57.04 44.95) (size 0.8) (drill 0.4) (layers "F.Cu" "B.Cu") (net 2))
 (segment (start 56.8275 44.7375) (end 57.04 44.95) (width 0.25) (layer "B.Cu") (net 2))
 (segment (start 53.1125 44.7375) (end 56.8275 44.7375) (width 0.25) (layer "B.Cu") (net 2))
 (segment (start 22.07 52.29) (end 24.06 54.28) (width 0.25) (layer "F.Cu") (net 1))
 (segment (start 30.18 35.81) (end 25.85 35.81) (width 0.25) (layer "F.Cu") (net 1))
 (segment (start 52.26 50.08) (end 51.2875 49.1075) (width 0.25) (layer "F.Cu") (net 1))
 (segment (start 22.07 39.59) (end 22.07 52.29) (width 0.25) (layer "F.Cu") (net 1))
 (segment (start 52.26 52.45) (end 52.26 50.08) (width 0.25) (layer "F.Cu") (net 1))
 (segment (start 25.85 35.81) (end 22.07 39.59) (width 0.25) (layer "F.Cu") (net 1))
 (segment (start 50.43 54.28) (end 52.26 52.45) (width 0.25) (layer "F.Cu") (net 1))
 (segment (start 24.06 54.28) (end 50.43 54.28) (width 0.25) (layer "F.Cu") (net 1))
 (segment (start 51.2875 49.1075) (end 51.2875 47.48) (width 0.25) (layer "F.Cu") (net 1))
 (segment (start 50.21 38.03) (end 51.2875 39.1075) (width 0.25) (layer "F.Cu") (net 10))
 (segment (start 38.18 35.79) (end 40.42 38.03) (width 0.25) (layer "F.Cu") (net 10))
 (segment (start 40.42 38.03) (end 50.21 38.03) (width 0.25) (layer "F.Cu") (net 10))
 (segment (start 51.2875 39.1075) (end 51.2875 43.08) (width 0.25) (layer "F.Cu") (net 10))
 (segment (start 36.45 35.79) (end 38.18 35.79) (width 0.25) (layer "F.Cu") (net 10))
 (segment (start 44.69 35.8) (end 45.54 34.95) (width 0.25) (layer "F.Cu") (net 6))
 (segment (start 42.22672 35.8) (end 44.69 35.8) (width 0.25) (layer "F.Cu") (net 6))
 (via (at 45.54 34.95) (size 0.8) (drill 0.4) (layers "F.Cu" "B.Cu") (free) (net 6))
 (segment (start 45.54 34.95) (end 45.54 31.17) (width 0.25) (layer "B.Cu") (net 6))
 (segment (start 45.54 31.17) (end 42.17 27.8) (width 0.25) (layer "B.Cu") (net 6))
 (segment (start 42.27836 32.52) (end 42.27836 31.73836) (width 0.25) (layer "F.Cu") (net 8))
 (segment (start 42.27836 31.73836) (end 41.45 30.91) (width 0.25) (layer "F.Cu") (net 8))
 (via (at 41.45 30.91) (size 0.8) (drill 0.4) (layers "F.Cu" "B.Cu") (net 8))
 (segment (start 38.02 29.53) (end 38.02 21.17) (width 0.25) (layer "B.Cu") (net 8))
 (segment (start 38.5 20.69) (end 42.06 20.69) (width 0.25) (layer "B.Cu") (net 8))
 (segment (start 39.4 30.91) (end 38.02 29.53) (width 0.25) (layer "B.Cu") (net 8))
 (segment (start 41.45 30.91) (end 39.4 30.91) (width 0.25) (layer "B.Cu") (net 8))
 (segment (start 42.33 20.96) (end 42.33 22.9) (width 0.25) (layer "B.Cu") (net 8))
 (segment (start 42.06 20.69) (end 42.33 20.96) (width 0.25) (layer "B.Cu") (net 8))
 (segment (start 38.02 21.17) (end 38.5 20.69) (width 0.25) (layer "B.Cu") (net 8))
 (segment (start 24.28 34.01) (end 23.83 34.01) (width 0.25) (layer "F.Cu") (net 14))
 (segment (start 40.58164 32.52) (end 38.99164 34.11) (width 0.25) (layer "F.Cu") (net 14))
 (segment (start 30.17 39.83) (end 27.42 39.83) (width 0.25) (layer "F.Cu") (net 14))
 (segment (start 38.99164 34.11) (end 24.38 34.11) (width 0.25) (layer "F.Cu") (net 14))
 (segment (start 24.38 34.11) (end 24.28 34.01) (width 0.25) (layer "F.Cu") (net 14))
 (segment (start 27.42 39.83) (end 27.25 39.66) (width 0.25) (layer "F.Cu") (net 14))
 (segment (start 23.83 34.01) (end 22.84 35) (width 0.25) (layer "F.Cu") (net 14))
 (via (at 22.84 35) (size 0.8) (drill 0.4) (layers "F.Cu" "B.Cu") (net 14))
 (via (at 27.25 39.66) (size 0.8) (drill 0.4) (layers "F.Cu" "B.Cu") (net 14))
 (segment (start 22.72 35.12) (end 22.84 35) (width 0.25) (layer "B.Cu") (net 14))
 (segment (start 25.87 39.66) (end 22.72 36.51) (width 0.25) (layer "B.Cu") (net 14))
 (segment (start 27.25 39.66) (end 25.87 39.66) (width 0.25) (layer "B.Cu") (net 14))
 (segment (start 22.72 36.51) (end 22.72 35.12) (width 0.25) (layer "B.Cu") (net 14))
 (segment (start 40.53 36.4) (end 41.39 37.26) (width 0.25) (layer "F.Cu") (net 7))
 (segment (start 37.6 38.65) (end 41.33 38.65) (width 0.25) (layer "F.Cu") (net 7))
 (segment (start 41.33 38.65) (end 41.52 38.84) (width 0.25) (layer "F.Cu") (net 7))
 (segment (start 40.53 35.8) (end 40.53 36.4) (width 0.25) (layer "F.Cu") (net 7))
 (segment (start 36.44 39.81) (end 37.6 38.65) (width 0.25) (layer "F.Cu") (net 7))
 (via (at 41.39 37.26) (size 0.8) (drill 0.4) (layers "F.Cu" "B.Cu") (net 7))
 (via (at 41.52 38.84) (size 0.8) (drill 0.4) (layers "F.Cu" "B.Cu") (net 7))
 (segment (start 41.52 37.39) (end 41.39 37.26) (width 0.25) (layer "B.Cu") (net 7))
 (segment (start 41.52 38.84) (end 41.52 37.39) (width 0.25) (layer "B.Cu") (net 7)))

